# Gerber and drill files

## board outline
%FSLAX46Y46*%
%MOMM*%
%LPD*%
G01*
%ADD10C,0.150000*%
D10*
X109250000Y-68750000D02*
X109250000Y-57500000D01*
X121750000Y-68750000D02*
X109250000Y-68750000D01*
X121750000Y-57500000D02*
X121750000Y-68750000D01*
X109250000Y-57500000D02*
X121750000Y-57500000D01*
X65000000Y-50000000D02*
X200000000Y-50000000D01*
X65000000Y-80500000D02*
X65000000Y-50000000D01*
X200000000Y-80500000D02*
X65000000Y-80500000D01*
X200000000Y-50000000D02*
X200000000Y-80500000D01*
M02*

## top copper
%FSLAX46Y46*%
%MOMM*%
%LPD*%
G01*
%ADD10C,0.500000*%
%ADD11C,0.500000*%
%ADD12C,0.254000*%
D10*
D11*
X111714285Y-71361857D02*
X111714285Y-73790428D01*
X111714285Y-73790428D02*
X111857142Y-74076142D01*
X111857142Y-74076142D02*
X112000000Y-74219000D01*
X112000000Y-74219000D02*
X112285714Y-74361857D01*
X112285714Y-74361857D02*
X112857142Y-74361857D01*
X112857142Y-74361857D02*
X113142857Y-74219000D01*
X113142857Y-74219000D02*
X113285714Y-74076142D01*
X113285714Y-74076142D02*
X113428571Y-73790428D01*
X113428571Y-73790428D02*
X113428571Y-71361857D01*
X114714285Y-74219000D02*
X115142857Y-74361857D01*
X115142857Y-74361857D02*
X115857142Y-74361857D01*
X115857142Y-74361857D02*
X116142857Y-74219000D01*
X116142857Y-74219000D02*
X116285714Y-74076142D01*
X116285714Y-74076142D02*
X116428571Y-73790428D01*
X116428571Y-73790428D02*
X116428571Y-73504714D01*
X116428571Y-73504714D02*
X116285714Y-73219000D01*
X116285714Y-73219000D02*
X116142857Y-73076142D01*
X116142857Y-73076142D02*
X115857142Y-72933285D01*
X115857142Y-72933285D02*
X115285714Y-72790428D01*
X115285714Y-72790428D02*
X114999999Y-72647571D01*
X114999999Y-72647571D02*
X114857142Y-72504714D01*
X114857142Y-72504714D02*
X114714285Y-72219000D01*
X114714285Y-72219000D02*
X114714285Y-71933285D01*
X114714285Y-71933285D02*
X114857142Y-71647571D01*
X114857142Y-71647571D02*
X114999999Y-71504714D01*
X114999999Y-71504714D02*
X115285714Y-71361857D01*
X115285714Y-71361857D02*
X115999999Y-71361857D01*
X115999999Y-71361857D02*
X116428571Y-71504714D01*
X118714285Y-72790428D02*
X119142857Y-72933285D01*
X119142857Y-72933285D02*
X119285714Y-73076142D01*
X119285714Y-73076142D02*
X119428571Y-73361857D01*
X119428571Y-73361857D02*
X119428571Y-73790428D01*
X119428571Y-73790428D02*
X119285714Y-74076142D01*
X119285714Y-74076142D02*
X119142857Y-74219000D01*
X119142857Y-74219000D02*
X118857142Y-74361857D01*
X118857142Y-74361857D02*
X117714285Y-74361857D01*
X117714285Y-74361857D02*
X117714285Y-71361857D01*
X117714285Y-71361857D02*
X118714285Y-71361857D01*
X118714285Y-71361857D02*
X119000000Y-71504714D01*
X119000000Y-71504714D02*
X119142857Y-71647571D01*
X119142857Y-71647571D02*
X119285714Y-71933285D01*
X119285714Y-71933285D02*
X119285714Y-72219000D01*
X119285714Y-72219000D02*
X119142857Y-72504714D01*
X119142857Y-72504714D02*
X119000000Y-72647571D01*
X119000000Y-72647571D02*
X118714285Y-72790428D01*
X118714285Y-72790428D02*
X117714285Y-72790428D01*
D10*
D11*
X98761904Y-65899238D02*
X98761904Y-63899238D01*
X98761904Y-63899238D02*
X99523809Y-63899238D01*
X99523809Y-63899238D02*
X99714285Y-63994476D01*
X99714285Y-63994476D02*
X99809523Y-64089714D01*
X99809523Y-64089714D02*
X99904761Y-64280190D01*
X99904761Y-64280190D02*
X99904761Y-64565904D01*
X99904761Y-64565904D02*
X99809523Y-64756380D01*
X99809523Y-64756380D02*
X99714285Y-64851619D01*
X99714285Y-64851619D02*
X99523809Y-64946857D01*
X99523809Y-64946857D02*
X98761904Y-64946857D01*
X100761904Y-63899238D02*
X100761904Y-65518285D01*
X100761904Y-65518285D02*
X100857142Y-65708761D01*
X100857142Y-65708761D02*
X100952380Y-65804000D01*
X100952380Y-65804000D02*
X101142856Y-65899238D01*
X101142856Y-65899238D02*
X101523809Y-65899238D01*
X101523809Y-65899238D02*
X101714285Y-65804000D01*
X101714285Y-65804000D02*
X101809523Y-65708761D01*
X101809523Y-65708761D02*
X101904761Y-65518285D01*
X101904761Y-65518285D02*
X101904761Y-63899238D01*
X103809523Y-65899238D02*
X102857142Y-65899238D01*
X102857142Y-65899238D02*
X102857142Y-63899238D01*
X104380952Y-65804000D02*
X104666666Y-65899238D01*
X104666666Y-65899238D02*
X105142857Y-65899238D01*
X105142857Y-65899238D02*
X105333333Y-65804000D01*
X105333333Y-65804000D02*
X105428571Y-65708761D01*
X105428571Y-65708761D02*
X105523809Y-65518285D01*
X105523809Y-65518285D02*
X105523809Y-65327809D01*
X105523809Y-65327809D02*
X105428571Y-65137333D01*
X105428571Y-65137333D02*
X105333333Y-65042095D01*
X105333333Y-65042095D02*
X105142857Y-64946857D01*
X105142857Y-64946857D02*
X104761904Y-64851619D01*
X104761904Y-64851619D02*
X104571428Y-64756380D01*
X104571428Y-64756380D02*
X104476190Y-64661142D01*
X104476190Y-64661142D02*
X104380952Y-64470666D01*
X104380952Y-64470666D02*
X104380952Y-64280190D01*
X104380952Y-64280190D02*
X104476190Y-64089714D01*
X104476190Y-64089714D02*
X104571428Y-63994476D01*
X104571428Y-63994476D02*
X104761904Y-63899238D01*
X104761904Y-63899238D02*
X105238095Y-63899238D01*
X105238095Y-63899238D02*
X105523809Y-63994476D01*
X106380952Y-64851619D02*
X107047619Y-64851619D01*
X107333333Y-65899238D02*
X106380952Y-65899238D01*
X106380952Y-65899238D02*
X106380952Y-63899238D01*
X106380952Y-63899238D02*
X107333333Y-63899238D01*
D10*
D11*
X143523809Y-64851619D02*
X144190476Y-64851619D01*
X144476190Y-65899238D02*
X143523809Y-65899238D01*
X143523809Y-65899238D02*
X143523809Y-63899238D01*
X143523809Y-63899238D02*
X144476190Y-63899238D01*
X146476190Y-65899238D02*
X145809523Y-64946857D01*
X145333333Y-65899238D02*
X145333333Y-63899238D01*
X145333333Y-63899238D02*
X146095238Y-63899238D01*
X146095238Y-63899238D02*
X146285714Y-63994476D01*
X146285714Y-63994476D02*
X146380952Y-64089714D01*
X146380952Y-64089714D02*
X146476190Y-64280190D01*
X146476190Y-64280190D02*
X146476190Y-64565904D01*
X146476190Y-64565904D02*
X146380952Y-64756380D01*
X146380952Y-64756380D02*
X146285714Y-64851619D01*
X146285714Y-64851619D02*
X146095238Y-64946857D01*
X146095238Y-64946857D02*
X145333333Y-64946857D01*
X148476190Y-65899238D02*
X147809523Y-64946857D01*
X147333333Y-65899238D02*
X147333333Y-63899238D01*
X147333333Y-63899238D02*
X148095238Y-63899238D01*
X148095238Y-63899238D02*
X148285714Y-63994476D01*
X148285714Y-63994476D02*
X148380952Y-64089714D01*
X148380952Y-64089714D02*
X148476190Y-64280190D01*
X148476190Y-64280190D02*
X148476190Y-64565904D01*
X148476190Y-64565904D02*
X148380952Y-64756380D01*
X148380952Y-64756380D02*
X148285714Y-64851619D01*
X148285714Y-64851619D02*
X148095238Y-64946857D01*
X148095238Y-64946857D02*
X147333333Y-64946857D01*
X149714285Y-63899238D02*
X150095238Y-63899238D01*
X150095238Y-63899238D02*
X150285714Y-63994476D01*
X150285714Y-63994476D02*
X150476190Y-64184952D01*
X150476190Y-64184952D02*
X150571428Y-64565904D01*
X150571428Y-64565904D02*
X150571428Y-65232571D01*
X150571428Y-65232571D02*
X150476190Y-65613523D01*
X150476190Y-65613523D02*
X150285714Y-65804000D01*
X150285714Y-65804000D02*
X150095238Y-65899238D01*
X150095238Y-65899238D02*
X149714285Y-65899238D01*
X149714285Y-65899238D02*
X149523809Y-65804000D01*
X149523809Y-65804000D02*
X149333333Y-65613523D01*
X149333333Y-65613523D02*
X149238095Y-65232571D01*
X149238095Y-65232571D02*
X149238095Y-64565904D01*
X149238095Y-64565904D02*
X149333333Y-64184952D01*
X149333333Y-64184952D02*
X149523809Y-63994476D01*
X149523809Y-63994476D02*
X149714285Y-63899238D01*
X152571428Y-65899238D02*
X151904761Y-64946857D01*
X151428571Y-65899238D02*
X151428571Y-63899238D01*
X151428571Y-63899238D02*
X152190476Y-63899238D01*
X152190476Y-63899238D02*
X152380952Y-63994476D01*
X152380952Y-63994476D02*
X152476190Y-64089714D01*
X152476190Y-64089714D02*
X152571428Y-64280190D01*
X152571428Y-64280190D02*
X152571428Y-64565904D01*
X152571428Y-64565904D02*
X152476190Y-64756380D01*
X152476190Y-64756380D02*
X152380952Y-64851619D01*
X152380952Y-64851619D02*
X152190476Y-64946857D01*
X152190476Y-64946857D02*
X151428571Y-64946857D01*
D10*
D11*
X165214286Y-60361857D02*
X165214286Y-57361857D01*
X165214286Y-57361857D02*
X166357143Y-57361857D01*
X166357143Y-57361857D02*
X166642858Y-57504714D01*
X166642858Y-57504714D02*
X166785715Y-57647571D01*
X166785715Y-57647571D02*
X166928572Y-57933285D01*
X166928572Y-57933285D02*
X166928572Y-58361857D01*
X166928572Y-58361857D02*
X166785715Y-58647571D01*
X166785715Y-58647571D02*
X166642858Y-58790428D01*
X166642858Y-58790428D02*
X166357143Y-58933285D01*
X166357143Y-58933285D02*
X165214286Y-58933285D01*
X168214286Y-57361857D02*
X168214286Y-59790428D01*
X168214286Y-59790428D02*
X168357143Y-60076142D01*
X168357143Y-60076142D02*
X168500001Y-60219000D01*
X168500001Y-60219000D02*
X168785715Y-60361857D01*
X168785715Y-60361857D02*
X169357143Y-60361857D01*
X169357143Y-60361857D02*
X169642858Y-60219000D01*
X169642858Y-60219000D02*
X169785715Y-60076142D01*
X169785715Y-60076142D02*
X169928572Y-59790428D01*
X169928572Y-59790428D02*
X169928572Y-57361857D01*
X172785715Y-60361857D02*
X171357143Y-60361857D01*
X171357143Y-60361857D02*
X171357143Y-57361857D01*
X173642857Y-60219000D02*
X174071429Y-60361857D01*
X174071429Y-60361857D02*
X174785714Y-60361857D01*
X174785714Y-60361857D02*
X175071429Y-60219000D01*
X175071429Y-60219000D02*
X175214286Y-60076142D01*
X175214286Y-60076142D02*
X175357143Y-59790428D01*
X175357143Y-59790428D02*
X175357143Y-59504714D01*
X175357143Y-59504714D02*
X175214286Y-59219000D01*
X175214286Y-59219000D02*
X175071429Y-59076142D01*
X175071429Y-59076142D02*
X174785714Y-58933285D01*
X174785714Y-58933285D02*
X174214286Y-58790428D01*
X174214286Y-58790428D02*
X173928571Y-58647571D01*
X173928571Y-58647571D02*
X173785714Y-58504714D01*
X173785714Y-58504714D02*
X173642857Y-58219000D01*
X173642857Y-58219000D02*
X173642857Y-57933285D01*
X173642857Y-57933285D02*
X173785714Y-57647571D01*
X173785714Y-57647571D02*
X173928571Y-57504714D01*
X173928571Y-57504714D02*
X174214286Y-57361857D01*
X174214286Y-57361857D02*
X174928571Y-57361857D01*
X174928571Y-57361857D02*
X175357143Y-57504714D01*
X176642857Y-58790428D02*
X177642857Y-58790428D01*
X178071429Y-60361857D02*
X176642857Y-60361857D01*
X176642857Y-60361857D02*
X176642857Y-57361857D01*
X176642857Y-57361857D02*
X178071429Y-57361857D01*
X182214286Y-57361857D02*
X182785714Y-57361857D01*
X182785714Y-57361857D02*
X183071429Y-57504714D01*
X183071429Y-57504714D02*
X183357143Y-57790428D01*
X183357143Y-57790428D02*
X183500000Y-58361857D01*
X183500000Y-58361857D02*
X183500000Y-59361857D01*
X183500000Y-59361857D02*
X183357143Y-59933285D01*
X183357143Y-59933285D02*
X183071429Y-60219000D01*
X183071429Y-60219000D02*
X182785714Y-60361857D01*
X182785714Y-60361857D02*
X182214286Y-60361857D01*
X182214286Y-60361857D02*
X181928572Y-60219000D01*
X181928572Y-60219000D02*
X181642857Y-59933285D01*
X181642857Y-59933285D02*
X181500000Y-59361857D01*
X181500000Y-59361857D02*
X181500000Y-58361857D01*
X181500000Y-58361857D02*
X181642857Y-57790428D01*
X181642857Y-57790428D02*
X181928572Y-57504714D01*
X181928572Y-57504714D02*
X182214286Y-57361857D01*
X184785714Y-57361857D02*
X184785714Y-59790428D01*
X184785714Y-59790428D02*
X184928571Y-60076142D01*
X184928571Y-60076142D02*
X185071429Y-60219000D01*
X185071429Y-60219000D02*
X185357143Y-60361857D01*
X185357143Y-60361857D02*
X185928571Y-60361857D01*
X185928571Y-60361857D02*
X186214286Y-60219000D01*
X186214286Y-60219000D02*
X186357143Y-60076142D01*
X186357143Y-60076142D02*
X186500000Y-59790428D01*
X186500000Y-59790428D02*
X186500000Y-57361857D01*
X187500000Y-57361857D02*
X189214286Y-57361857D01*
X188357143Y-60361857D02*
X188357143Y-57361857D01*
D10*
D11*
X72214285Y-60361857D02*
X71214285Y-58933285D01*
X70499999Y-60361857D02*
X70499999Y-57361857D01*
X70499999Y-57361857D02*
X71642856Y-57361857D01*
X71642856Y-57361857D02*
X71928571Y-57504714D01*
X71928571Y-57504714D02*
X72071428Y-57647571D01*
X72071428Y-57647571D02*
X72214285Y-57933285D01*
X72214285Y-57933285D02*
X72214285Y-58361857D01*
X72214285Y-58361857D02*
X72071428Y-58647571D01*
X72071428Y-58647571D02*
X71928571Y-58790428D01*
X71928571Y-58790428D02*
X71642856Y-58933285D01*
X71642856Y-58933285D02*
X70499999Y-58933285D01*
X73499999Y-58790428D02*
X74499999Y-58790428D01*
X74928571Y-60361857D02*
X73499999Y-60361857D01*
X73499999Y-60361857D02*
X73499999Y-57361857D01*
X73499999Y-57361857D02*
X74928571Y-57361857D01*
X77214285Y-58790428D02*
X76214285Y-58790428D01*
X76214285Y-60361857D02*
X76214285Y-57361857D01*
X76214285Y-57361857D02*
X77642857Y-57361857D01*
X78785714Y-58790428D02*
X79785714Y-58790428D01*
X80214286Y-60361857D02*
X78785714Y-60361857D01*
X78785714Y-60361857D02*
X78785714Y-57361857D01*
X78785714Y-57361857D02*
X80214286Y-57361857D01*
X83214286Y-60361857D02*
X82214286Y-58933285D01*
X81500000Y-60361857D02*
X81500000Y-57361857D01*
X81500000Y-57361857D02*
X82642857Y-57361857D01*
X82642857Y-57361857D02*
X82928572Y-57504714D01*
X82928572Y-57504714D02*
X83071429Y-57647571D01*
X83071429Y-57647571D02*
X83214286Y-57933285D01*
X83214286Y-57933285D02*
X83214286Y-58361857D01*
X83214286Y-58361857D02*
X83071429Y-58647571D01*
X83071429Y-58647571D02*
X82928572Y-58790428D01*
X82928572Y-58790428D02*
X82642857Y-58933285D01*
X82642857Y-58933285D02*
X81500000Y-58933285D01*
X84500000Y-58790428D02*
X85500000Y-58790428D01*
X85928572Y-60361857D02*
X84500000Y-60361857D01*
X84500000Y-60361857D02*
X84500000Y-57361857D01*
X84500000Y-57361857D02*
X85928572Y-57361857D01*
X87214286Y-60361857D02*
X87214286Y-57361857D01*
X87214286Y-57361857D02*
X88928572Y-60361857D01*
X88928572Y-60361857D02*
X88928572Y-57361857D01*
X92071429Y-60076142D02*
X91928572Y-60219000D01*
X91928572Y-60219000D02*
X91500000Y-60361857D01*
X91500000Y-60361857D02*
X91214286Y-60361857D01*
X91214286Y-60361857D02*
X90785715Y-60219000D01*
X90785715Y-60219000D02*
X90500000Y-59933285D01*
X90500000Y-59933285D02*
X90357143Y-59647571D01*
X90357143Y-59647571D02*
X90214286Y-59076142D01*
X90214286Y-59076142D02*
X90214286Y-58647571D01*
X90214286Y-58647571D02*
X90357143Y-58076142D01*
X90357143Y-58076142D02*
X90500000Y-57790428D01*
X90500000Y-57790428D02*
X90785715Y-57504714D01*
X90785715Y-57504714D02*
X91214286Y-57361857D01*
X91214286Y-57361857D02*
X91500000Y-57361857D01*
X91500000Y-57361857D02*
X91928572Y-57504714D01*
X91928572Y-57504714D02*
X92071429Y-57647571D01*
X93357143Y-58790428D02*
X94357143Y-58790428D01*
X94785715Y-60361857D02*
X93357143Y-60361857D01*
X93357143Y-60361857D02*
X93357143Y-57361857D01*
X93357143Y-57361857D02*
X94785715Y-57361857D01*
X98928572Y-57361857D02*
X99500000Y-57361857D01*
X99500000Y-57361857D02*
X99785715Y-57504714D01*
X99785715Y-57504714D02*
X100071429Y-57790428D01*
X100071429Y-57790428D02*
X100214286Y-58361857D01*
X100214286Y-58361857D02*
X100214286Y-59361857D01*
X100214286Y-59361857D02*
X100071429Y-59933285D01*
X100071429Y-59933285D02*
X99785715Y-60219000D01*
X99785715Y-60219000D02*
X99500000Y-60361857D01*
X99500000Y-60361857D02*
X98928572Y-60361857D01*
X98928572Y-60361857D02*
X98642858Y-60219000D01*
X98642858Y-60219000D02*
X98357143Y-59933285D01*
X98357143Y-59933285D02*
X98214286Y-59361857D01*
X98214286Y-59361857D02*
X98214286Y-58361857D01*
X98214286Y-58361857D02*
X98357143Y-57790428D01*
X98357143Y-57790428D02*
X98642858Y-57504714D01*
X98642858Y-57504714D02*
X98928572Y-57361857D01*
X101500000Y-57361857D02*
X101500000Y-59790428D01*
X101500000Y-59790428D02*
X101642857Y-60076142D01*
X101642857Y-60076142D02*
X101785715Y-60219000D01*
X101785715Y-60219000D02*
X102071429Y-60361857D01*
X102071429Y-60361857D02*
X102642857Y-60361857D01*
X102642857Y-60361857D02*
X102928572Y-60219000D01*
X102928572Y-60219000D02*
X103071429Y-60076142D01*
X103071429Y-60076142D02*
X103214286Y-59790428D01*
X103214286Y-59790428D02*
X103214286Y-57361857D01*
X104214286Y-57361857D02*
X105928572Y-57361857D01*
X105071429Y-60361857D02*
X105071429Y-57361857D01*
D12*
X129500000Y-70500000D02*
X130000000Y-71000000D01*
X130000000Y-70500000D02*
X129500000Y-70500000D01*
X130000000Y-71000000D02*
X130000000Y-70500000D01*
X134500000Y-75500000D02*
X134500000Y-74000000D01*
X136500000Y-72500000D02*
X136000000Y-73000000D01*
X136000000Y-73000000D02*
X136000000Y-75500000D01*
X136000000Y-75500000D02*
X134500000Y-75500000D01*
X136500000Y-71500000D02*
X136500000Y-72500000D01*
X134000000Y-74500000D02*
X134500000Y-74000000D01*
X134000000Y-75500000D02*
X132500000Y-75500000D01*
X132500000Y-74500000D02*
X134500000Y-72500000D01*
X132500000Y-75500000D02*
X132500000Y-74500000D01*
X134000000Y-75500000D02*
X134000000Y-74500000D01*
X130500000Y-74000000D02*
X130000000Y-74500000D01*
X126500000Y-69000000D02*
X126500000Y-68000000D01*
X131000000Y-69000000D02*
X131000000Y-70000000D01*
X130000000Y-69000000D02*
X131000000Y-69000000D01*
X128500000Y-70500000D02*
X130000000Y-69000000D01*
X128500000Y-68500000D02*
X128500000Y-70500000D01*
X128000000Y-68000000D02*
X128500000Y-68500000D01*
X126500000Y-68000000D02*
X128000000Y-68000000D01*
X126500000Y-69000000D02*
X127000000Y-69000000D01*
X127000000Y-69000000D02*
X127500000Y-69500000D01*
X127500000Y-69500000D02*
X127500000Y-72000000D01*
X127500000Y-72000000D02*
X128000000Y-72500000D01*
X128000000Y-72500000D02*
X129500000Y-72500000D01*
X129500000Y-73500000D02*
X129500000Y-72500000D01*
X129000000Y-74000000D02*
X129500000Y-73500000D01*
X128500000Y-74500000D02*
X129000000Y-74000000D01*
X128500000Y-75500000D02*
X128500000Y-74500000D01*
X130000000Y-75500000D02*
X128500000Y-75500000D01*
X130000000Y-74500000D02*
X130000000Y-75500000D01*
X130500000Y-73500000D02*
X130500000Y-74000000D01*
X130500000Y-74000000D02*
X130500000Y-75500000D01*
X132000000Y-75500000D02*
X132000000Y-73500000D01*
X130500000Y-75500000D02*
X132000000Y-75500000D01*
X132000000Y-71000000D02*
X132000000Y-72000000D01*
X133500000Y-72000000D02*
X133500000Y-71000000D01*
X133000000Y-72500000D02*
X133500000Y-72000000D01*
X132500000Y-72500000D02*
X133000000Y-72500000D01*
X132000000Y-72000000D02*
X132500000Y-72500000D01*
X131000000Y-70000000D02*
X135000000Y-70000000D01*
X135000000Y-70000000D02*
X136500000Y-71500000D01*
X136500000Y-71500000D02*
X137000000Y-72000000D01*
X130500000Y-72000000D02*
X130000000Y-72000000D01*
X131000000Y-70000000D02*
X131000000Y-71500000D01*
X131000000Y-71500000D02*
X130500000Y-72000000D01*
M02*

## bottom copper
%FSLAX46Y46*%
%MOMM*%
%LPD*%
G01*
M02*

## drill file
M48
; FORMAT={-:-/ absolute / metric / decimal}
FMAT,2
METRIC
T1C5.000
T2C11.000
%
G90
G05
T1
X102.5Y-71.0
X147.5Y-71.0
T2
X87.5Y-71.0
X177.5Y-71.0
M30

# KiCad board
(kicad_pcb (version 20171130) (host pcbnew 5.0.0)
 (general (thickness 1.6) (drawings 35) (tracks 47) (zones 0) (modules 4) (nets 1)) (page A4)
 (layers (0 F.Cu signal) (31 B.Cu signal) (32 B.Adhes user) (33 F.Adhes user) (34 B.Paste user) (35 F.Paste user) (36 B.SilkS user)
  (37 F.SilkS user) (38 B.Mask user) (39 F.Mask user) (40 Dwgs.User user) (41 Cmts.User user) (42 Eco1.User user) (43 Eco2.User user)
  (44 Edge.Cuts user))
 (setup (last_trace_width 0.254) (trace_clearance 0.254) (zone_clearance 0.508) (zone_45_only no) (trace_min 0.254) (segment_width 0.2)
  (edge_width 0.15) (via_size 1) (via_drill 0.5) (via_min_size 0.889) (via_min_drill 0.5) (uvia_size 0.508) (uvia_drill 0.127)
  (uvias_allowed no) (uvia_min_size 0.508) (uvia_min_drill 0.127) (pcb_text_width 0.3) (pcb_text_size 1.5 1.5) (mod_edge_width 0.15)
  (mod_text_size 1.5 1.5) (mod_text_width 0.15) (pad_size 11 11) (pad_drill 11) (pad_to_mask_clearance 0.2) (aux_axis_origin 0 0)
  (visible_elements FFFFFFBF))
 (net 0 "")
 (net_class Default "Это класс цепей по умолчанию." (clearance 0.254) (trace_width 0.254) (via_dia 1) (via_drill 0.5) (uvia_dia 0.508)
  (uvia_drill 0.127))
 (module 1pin (layer F.Cu) (at 87.5 71)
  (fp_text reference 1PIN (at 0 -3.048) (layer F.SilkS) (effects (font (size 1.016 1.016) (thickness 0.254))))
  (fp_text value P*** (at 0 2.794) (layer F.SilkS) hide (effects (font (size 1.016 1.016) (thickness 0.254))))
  (pad "" np_thru_hole circle (at 0 0) (size 11 11) (drill 11) (layers *.Cu *.Mask F.SilkS)))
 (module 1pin (layer F.Cu) (at 177.5 71)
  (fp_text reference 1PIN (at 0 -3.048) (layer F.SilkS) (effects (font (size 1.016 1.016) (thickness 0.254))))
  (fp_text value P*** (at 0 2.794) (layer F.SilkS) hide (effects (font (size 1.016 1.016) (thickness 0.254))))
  (pad "" np_thru_hole circle (at 0 0) (size 11 11) (drill 11) (layers *.Cu *.Mask F.SilkS)))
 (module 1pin (layer F.Cu) (at 102.5 71)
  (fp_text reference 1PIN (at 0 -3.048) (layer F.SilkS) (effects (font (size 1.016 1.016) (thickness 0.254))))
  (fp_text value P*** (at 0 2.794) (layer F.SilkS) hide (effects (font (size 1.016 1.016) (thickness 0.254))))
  (pad "" np_thru_hole circle (at 0 0) (size 5 5) (drill 5) (layers *.Cu *.Mask F.SilkS)))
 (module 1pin (layer F.Cu) (at 147.5 71)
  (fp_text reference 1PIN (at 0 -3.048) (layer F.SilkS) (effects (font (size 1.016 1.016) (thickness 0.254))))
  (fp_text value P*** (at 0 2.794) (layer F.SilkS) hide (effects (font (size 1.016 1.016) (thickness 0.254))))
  (pad "" np_thru_hole circle (at 0 0) (size 5 5) (drill 5) (layers *.Cu *.Mask F.SilkS)))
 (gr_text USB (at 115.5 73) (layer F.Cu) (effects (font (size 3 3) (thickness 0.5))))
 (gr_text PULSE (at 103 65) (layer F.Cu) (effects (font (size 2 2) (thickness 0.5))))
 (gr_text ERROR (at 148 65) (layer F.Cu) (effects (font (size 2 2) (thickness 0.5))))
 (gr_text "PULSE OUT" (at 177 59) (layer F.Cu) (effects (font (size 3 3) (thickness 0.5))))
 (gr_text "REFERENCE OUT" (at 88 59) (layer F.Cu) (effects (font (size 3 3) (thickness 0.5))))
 (gr_line (start 109.25 68.75) (end 109.25 57.5) (angle 90) (layer Edge.Cuts) (width 0.15))
 (gr_line (start 121.75 68.75) (end 109.25 68.75) (angle 90) (layer Edge.Cuts) (width 0.15))
 (gr_line (start 121.75 57.5) (end 121.75 68.75) (angle 90) (layer Edge.Cuts) (width 0.15))
 (gr_line (start 109.25 57.5) (end 121.75 57.5) (angle 90) (layer Edge.Cuts) (width 0.15))
 (gr_line (start 65 50) (end 200 50) (angle 90) (layer Edge.Cuts) (width 0.15))
 (gr_line (start 65 80.5) (end 65 50) (angle 90) (layer Edge.Cuts) (width 0.15))
 (gr_line (start 200 80.5) (end 65 80.5) (angle 90) (layer Edge.Cuts) (width 0.15))
 (gr_line (start 200 50) (end 200 80.5) (angle 90) (layer Edge.Cuts) (width 0.15))
 (segment (start 129.5 70.5) (end 130 71) (width 0.254) (layer F.Cu) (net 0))
 (segment (start 130 70.5) (end 129.5 70.5) (width 0.254) (layer F.Cu) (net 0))
 (segment (start 130 71) (end 130 70.5) (width 0.254) (layer F.Cu) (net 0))
 (segment (start 134.5 75.5) (end 134.5 74) (width 0.254) (layer F.Cu) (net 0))
 (segment (start 136.5 72.5) (end 136 73) (width 0.254) (layer F.Cu) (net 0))
 (segment (start 136 73) (end 136 75.5) (width 0.254) (layer F.Cu) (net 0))
 (segment (start 136 75.5) (end 134.5 75.5) (width 0.254) (layer F.Cu) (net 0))
 (segment (start 136.5 71.5) (end 136.5 72.5) (width 0.254) (layer F.Cu) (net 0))
 (segment (start 134 74.5) (end 134.5 74) (width 0.254) (layer F.Cu) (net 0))
 (segment (start 134 75.5) (end 132.5 75.5) (width 0.254) (layer F.Cu) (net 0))
 (segment (start 132.5 74.5) (end 134.5 72.5) (width 0.254) (layer F.Cu) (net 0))
 (segment (start 132.5 75.5) (end 132.5 74.5) (width 0.254) (layer F.Cu) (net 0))
 (segment (start 134 75.5) (end 134 74.5) (width 0.254) (layer F.Cu) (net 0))
 (segment (start 130.5 74) (end 130 74.5) (width 0.254) (layer F.Cu) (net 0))
 (segment (start 126.5 69) (end 126.5 68) (width 0.254) (layer F.Cu) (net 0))
 (segment (start 131 69) (end 131 70) (width 0.254) (layer F.Cu) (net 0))
 (segment (start 130 69) (end 131 69) (width 0.254) (layer F.Cu) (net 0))
 (segment (start 128.5 70.5) (end 130 69) (width 0.254) (layer F.Cu) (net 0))
 (segment (start 128.5 68.5) (end 128.5 70.5) (width 0.254) (layer F.Cu) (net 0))
 (segment (start 128 68) (end 128.5 68.5) (width 0.254) (layer F.Cu) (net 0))
 (segment (start 126.5 68) (end 128 68) (width 0.254) (layer F.Cu) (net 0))
 (segment (start 126.5 69) (end 127 69) (width 0.254) (layer F.Cu) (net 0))
 (segment (start 127 69) (end 127.5 69.5) (width 0.254) (layer F.Cu) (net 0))
 (segment (start 127.5 69.5) (end 127.5 72) (width 0.254) (layer F.Cu) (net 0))
 (segment (start 127.5 72) (end 128 72.5) (width 0.254) (layer F.Cu) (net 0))
 (segment (start 128 72.5) (end 129.5 72.5) (width 0.254) (layer F.Cu) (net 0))
 (segment (start 129.5 73.5) (end 129.5 72.5) (width 0.254) (layer F.Cu) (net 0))
 (segment (start 129 74) (end 129.5 73.5) (width 0.254) (layer F.Cu) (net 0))
 (segment (start 128.5 74.5) (end 129 74) (width 0.254) (layer F.Cu) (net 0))
 (segment (start 128.5 75.5) (end 128.5 74.5) (width 0.254) (layer F.Cu) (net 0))
 (segment (start 130 75.5) (end 128.5 75.5) (width 0.254) (layer F.Cu) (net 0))
 (segment (start 130 74.5) (end 130 75.5) (width 0.254) (layer F.Cu) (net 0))
 (segment (start 130.5 73.5) (end 130.5 74) (width 0.254) (layer F.Cu) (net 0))
 (segment (start 130.5 74) (end 130.5 75.5) (width 0.254) (layer F.Cu) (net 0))
 (segment (start 132 75.5) (end 132 73.5) (width 0.254) (layer F.Cu) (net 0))
 (segment (start 130.5 75.5) (end 132 75.5) (width 0.254) (layer F.Cu) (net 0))
 (segment (start 132 71) (end 132 72) (width 0.254) (layer F.Cu) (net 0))
 (segment (start 133.5 72) (end 133.5 71) (width 0.254) (layer F.Cu) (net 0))
 (segment (start 133 72.5) (end 133.5 72) (width 0.254) (layer F.Cu) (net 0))
 (segment (start 132.5 72.5) (end 133 72.5) (width 0.254) (layer F.Cu) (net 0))
 (segment (start 132 72) (end 132.5 72.5) (width 0.254) (layer F.Cu) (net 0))
 (segment (start 131 70) (end 135 70) (width 0.254) (layer F.Cu) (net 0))
 (segment (start 135 70) (end 136.5 71.5) (width 0.254) (layer F.Cu) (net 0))
 (segment (start 136.5 71.5) (end 137 72) (width 0.254) (layer F.Cu) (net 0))
 (segment (start 130.5 72) (end 130 72) (width 0.254) (layer F.Cu) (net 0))
 (segment (start 131 70) (end 131 71.5) (width 0.254) (layer F.Cu) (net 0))
 (segment (start 131 71.5) (end 130.5 72) (width 0.254) (layer F.Cu) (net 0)))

